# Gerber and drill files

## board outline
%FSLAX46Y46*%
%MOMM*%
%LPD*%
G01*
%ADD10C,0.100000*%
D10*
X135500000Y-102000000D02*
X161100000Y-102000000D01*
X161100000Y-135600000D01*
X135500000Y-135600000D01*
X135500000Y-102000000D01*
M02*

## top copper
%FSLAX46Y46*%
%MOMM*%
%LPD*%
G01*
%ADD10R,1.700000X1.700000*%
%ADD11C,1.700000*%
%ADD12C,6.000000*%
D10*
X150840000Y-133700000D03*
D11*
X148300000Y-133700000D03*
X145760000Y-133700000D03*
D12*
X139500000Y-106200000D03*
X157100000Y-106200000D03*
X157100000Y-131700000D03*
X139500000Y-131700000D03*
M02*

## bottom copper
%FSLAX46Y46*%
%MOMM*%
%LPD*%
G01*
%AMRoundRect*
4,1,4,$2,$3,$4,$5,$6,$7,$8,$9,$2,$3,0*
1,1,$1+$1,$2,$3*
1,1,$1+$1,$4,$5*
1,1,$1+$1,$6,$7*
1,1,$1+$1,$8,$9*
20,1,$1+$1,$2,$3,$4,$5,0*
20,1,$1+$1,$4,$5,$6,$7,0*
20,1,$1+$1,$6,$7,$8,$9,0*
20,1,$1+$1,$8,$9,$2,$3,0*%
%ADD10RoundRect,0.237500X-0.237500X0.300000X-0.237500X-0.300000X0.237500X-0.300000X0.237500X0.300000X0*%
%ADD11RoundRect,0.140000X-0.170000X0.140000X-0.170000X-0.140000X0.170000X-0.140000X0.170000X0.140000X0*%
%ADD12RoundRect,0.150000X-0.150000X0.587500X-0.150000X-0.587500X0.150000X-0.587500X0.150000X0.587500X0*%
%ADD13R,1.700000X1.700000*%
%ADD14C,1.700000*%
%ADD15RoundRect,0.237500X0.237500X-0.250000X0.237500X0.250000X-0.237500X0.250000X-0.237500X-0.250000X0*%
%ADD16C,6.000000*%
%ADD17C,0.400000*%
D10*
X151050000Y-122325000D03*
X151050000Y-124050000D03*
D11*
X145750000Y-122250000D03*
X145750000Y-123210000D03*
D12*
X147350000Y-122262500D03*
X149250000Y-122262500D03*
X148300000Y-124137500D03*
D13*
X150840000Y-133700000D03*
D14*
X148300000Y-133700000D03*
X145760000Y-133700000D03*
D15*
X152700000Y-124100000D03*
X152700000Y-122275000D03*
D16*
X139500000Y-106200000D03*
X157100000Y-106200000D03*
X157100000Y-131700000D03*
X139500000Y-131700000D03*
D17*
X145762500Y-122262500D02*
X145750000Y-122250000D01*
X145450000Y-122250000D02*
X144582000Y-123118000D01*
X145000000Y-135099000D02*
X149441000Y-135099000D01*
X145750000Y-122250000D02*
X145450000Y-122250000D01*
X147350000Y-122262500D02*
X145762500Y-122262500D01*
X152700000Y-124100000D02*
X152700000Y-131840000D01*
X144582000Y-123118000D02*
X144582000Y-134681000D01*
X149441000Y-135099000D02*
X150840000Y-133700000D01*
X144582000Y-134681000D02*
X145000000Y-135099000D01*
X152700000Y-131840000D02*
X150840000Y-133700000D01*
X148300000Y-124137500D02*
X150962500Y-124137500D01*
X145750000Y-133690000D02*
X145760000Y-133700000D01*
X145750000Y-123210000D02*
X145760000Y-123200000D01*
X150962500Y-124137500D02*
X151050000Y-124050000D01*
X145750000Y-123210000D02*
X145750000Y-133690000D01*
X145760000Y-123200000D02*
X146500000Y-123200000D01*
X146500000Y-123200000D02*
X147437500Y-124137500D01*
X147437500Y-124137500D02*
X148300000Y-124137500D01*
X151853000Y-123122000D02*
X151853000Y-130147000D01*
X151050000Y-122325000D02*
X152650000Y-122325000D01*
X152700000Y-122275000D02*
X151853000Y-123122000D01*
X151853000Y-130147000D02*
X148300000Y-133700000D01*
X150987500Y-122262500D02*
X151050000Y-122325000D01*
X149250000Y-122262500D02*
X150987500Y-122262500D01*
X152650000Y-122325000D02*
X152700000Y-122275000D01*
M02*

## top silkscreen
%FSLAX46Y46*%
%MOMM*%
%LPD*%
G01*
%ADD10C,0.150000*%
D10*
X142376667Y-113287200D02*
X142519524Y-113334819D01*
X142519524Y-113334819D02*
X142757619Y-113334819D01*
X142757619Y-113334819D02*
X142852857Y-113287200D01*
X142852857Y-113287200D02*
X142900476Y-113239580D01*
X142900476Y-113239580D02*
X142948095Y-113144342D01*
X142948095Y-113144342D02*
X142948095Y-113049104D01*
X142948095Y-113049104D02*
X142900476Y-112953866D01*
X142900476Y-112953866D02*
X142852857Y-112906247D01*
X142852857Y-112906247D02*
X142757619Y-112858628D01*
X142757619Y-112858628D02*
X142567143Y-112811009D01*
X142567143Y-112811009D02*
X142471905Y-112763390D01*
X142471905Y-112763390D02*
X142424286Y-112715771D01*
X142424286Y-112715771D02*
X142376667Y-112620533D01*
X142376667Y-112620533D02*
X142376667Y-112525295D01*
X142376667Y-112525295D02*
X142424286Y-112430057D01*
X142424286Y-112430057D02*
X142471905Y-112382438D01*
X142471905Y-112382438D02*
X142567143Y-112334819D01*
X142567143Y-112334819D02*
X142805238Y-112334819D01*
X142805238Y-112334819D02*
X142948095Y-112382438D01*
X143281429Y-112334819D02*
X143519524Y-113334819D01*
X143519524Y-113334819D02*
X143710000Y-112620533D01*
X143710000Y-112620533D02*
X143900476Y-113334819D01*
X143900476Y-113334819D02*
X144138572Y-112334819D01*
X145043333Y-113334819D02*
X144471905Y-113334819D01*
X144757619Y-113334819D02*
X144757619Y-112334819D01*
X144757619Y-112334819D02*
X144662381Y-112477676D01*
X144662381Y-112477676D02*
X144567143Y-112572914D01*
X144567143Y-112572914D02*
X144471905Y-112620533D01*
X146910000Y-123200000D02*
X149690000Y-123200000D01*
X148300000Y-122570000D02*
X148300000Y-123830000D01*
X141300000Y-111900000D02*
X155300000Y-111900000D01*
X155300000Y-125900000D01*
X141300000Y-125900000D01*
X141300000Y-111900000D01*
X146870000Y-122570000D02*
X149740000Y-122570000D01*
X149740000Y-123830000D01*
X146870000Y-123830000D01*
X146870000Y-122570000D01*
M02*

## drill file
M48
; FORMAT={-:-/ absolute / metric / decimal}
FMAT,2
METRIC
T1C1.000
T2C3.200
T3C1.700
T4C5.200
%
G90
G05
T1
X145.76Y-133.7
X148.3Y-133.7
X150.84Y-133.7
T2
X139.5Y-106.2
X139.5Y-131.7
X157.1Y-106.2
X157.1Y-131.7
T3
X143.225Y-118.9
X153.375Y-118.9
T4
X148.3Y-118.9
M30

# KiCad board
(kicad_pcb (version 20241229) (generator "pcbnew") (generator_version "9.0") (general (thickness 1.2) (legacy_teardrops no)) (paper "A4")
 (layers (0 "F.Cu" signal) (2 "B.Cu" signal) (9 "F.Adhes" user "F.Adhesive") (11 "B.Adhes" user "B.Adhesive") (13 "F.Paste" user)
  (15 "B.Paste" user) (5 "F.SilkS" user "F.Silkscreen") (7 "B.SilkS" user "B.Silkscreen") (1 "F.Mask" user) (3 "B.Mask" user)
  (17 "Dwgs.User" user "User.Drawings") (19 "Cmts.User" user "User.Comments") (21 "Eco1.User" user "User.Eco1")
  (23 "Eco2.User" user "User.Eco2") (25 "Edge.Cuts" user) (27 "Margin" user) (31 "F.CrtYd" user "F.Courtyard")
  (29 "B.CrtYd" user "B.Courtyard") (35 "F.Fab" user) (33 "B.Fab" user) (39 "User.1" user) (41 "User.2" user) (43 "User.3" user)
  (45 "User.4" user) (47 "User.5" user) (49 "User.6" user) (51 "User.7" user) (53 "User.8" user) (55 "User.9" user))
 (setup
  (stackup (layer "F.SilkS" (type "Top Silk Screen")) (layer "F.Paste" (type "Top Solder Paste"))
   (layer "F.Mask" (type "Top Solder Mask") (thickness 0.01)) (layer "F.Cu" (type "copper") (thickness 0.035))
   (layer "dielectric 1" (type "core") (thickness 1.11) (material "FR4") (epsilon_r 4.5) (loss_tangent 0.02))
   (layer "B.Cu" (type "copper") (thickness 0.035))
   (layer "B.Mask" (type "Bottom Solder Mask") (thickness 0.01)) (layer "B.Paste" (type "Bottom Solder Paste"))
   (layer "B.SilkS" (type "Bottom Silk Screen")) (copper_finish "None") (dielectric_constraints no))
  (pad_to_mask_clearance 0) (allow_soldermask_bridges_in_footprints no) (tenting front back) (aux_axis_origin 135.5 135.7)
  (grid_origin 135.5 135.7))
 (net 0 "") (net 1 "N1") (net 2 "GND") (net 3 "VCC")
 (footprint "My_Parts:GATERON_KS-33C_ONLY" (layer "F.Cu") (at 148.3 118.9)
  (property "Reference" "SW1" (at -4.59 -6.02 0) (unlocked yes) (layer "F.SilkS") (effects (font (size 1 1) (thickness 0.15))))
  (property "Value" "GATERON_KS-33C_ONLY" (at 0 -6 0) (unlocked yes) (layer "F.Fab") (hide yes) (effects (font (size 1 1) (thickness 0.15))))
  (fp_line (start -1.39 4.3) (end 1.39 4.3) (stroke (width 0.15) (type solid)) (layer "F.SilkS"))
  (fp_line (start 0 3.67) (end 0 4.93) (stroke (width 0.15) (type solid)) (layer "F.SilkS"))
  (fp_rect (start -7 -7) (end 7 7) (stroke (width 0.15) (type solid)) (fill no) (layer "F.SilkS"))
  (fp_rect (start -1.43 3.67) (end 1.44 4.93) (stroke (width 0.15) (type default)) (fill no) (layer "F.SilkS"))
  (pad "" np_thru_hole circle (at -5.075 0) (size 1.7 1.7) (drill 1.7) (layers "*.Cu" "*.Mask"))
  (pad "" np_thru_hole circle (at 0 0) (size 5.2 5.2) (drill 5.2) (layers "*.Cu" "*.Mask"))
  (pad "" np_thru_hole circle (at 5.075 0) (size 1.7 1.7) (drill 1.7) (layers "*.Cu" "*.Mask")))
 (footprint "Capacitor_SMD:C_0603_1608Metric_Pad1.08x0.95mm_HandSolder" (layer "B.Cu") (at 151.05 123.1875 -90)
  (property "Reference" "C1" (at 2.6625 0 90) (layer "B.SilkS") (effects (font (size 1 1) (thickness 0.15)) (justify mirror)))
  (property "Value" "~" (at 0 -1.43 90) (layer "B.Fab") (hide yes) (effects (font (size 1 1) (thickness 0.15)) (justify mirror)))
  (pad "1" smd roundrect (at -0.8625 0 270) (size 1.075 0.95) (layers "B.Cu" "B.Mask" "B.Paste") (roundrect_rratio 0.25) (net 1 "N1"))
  (pad "2" smd roundrect (at 0.8625 0 270) (size 1.075 0.95) (layers "B.Cu" "B.Mask" "B.Paste") (roundrect_rratio 0.25) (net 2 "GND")))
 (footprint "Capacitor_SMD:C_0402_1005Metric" (layer "B.Cu") (at 145.75 122.73 -90)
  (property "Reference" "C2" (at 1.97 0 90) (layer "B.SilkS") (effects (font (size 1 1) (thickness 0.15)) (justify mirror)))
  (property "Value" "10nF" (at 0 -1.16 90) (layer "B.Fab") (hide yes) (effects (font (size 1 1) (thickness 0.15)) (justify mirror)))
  (pad "1" smd roundrect (at -0.48 0 270) (size 0.56 0.62) (layers "B.Cu" "B.Mask" "B.Paste") (roundrect_rratio 0.25) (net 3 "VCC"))
  (pad "2" smd roundrect (at 0.48 0 270) (size 0.56 0.62) (layers "B.Cu" "B.Mask" "B.Paste") (roundrect_rratio 0.25) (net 2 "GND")))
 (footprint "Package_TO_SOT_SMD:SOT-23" (layer "B.Cu") (at 148.3 123.2 -90)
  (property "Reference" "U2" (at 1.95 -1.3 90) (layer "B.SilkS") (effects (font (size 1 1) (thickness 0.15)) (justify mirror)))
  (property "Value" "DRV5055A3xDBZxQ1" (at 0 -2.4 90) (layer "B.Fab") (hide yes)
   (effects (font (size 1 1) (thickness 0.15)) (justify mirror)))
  (pad "1" smd roundrect (at -0.9375 0.95 270) (size 1.475 0.6) (layers "B.Cu" "B.Mask" "B.Paste") (roundrect_rratio 0.25) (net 3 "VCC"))
  (pad "2" smd roundrect (at -0.9375 -0.95 270) (size 1.475 0.6) (layers "B.Cu" "B.Mask" "B.Paste") (roundrect_rratio 0.25) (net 1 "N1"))
  (pad "3" smd roundrect (at 0.9375 0 270) (size 1.475 0.6) (layers "B.Cu" "B.Mask" "B.Paste") (roundrect_rratio 0.25) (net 2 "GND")))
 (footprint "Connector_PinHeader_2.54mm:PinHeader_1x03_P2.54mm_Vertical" (layer "B.Cu") (at 150.84 133.7 90)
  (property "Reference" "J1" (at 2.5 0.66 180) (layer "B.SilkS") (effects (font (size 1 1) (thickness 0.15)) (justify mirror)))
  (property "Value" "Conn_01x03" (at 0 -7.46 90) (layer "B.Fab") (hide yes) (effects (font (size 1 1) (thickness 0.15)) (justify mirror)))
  (pad "1" thru_hole rect (at 0 0 90) (size 1.7 1.7) (drill 1) (layers "*.Cu" "*.Mask") (remove_unused_layers no) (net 3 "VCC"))
  (pad "2" thru_hole circle (at 0 -2.54 90) (size 1.7 1.7) (drill 1) (layers "*.Cu" "*.Mask") (remove_unused_layers no) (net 1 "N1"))
  (pad "3" thru_hole circle (at 0 -5.08 90) (size 1.7 1.7) (drill 1) (layers "*.Cu" "*.Mask") (remove_unused_layers no) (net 2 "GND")))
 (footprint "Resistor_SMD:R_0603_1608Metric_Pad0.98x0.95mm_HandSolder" (layer "B.Cu") (at 152.7 123.1875 90)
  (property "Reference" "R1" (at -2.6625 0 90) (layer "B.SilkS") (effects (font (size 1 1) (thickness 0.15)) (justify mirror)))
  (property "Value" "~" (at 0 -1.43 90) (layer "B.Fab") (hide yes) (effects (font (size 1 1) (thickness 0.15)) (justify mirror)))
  (pad "1" smd roundrect (at -0.9125 0 90) (size 0.975 0.95) (layers "B.Cu" "B.Mask" "B.Paste") (roundrect_rratio 0.25) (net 3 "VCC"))
  (pad "2" smd roundrect (at 0.9125 0 90) (size 0.975 0.95) (layers "B.Cu" "B.Mask" "B.Paste") (roundrect_rratio 0.25) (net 1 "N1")))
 (gr_rect (start 135.5 102) (end 161.1 135.6) (stroke (width 0.1) (type solid)) (fill no) (layer "Edge.Cuts"))
 (via (at 139.5 106.2) (size 6) (drill 3.2) (layers "F.Cu" "B.Cu") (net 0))
 (via (at 157.1 106.2) (size 6) (drill 3.2) (layers "F.Cu" "B.Cu") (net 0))
 (via (at 157.1 131.7) (size 6) (drill 3.2) (layers "F.Cu" "B.Cu") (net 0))
 (via (at 139.5 131.7) (size 6) (drill 3.2) (layers "F.Cu" "B.Cu") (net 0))
 (segment (start 145.7625 122.2625) (end 145.75 122.25) (width 0.4) (layer "B.Cu") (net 3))
 (segment (start 145.45 122.25) (end 144.582 123.118) (width 0.4) (layer "B.Cu") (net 3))
 (segment (start 145 135.099) (end 149.441 135.099) (width 0.4) (layer "B.Cu") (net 3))
 (segment (start 145.75 122.25) (end 145.45 122.25) (width 0.4) (layer "B.Cu") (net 3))
 (segment (start 147.35 122.2625) (end 145.7625 122.2625) (width 0.4) (layer "B.Cu") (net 3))
 (segment (start 152.7 124.1) (end 152.7 131.84) (width 0.4) (layer "B.Cu") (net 3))
 (segment (start 144.582 123.118) (end 144.582 134.681) (width 0.4) (layer "B.Cu") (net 3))
 (segment (start 149.441 135.099) (end 150.84 133.7) (width 0.4) (layer "B.Cu") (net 3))
 (segment (start 144.582 134.681) (end 145 135.099) (width 0.4) (layer "B.Cu") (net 3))
 (segment (start 152.7 131.84) (end 150.84 133.7) (width 0.4) (layer "B.Cu") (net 3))
 (segment (start 148.3 124.1375) (end 150.9625 124.1375) (width 0.4) (layer "B.Cu") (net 2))
 (segment (start 145.75 133.69) (end 145.76 133.7) (width 0.4) (layer "B.Cu") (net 2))
 (segment (start 145.75 123.21) (end 145.76 123.2) (width 0.4) (layer "B.Cu") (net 2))
 (segment (start 150.9625 124.1375) (end 151.05 124.05) (width 0.4) (layer "B.Cu") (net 2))
 (segment (start 145.75 123.21) (end 145.75 133.69) (width 0.4) (layer "B.Cu") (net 2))
 (segment (start 145.76 123.2) (end 146.5 123.2) (width 0.4) (layer "B.Cu") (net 2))
 (segment (start 146.5 123.2) (end 147.4375 124.1375) (width 0.4) (layer "B.Cu") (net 2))
 (segment (start 147.4375 124.1375) (end 148.3 124.1375) (width 0.4) (layer "B.Cu") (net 2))
 (segment (start 151.853 123.122) (end 151.853 130.147) (width 0.4) (layer "B.Cu") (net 1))
 (segment (start 151.05 122.325) (end 152.65 122.325) (width 0.4) (layer "B.Cu") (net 1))
 (segment (start 152.7 122.275) (end 151.853 123.122) (width 0.4) (layer "B.Cu") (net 1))
 (segment (start 151.853 130.147) (end 148.3 133.7) (width 0.4) (layer "B.Cu") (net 1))
 (segment (start 150.9875 122.2625) (end 151.05 122.325) (width 0.4) (layer "B.Cu") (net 1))
 (segment (start 149.25 122.2625) (end 150.9875 122.2625) (width 0.4) (layer "B.Cu") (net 1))
 (segment (start 152.65 122.325) (end 152.7 122.275) (width 0.4) (layer "B.Cu") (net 1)))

